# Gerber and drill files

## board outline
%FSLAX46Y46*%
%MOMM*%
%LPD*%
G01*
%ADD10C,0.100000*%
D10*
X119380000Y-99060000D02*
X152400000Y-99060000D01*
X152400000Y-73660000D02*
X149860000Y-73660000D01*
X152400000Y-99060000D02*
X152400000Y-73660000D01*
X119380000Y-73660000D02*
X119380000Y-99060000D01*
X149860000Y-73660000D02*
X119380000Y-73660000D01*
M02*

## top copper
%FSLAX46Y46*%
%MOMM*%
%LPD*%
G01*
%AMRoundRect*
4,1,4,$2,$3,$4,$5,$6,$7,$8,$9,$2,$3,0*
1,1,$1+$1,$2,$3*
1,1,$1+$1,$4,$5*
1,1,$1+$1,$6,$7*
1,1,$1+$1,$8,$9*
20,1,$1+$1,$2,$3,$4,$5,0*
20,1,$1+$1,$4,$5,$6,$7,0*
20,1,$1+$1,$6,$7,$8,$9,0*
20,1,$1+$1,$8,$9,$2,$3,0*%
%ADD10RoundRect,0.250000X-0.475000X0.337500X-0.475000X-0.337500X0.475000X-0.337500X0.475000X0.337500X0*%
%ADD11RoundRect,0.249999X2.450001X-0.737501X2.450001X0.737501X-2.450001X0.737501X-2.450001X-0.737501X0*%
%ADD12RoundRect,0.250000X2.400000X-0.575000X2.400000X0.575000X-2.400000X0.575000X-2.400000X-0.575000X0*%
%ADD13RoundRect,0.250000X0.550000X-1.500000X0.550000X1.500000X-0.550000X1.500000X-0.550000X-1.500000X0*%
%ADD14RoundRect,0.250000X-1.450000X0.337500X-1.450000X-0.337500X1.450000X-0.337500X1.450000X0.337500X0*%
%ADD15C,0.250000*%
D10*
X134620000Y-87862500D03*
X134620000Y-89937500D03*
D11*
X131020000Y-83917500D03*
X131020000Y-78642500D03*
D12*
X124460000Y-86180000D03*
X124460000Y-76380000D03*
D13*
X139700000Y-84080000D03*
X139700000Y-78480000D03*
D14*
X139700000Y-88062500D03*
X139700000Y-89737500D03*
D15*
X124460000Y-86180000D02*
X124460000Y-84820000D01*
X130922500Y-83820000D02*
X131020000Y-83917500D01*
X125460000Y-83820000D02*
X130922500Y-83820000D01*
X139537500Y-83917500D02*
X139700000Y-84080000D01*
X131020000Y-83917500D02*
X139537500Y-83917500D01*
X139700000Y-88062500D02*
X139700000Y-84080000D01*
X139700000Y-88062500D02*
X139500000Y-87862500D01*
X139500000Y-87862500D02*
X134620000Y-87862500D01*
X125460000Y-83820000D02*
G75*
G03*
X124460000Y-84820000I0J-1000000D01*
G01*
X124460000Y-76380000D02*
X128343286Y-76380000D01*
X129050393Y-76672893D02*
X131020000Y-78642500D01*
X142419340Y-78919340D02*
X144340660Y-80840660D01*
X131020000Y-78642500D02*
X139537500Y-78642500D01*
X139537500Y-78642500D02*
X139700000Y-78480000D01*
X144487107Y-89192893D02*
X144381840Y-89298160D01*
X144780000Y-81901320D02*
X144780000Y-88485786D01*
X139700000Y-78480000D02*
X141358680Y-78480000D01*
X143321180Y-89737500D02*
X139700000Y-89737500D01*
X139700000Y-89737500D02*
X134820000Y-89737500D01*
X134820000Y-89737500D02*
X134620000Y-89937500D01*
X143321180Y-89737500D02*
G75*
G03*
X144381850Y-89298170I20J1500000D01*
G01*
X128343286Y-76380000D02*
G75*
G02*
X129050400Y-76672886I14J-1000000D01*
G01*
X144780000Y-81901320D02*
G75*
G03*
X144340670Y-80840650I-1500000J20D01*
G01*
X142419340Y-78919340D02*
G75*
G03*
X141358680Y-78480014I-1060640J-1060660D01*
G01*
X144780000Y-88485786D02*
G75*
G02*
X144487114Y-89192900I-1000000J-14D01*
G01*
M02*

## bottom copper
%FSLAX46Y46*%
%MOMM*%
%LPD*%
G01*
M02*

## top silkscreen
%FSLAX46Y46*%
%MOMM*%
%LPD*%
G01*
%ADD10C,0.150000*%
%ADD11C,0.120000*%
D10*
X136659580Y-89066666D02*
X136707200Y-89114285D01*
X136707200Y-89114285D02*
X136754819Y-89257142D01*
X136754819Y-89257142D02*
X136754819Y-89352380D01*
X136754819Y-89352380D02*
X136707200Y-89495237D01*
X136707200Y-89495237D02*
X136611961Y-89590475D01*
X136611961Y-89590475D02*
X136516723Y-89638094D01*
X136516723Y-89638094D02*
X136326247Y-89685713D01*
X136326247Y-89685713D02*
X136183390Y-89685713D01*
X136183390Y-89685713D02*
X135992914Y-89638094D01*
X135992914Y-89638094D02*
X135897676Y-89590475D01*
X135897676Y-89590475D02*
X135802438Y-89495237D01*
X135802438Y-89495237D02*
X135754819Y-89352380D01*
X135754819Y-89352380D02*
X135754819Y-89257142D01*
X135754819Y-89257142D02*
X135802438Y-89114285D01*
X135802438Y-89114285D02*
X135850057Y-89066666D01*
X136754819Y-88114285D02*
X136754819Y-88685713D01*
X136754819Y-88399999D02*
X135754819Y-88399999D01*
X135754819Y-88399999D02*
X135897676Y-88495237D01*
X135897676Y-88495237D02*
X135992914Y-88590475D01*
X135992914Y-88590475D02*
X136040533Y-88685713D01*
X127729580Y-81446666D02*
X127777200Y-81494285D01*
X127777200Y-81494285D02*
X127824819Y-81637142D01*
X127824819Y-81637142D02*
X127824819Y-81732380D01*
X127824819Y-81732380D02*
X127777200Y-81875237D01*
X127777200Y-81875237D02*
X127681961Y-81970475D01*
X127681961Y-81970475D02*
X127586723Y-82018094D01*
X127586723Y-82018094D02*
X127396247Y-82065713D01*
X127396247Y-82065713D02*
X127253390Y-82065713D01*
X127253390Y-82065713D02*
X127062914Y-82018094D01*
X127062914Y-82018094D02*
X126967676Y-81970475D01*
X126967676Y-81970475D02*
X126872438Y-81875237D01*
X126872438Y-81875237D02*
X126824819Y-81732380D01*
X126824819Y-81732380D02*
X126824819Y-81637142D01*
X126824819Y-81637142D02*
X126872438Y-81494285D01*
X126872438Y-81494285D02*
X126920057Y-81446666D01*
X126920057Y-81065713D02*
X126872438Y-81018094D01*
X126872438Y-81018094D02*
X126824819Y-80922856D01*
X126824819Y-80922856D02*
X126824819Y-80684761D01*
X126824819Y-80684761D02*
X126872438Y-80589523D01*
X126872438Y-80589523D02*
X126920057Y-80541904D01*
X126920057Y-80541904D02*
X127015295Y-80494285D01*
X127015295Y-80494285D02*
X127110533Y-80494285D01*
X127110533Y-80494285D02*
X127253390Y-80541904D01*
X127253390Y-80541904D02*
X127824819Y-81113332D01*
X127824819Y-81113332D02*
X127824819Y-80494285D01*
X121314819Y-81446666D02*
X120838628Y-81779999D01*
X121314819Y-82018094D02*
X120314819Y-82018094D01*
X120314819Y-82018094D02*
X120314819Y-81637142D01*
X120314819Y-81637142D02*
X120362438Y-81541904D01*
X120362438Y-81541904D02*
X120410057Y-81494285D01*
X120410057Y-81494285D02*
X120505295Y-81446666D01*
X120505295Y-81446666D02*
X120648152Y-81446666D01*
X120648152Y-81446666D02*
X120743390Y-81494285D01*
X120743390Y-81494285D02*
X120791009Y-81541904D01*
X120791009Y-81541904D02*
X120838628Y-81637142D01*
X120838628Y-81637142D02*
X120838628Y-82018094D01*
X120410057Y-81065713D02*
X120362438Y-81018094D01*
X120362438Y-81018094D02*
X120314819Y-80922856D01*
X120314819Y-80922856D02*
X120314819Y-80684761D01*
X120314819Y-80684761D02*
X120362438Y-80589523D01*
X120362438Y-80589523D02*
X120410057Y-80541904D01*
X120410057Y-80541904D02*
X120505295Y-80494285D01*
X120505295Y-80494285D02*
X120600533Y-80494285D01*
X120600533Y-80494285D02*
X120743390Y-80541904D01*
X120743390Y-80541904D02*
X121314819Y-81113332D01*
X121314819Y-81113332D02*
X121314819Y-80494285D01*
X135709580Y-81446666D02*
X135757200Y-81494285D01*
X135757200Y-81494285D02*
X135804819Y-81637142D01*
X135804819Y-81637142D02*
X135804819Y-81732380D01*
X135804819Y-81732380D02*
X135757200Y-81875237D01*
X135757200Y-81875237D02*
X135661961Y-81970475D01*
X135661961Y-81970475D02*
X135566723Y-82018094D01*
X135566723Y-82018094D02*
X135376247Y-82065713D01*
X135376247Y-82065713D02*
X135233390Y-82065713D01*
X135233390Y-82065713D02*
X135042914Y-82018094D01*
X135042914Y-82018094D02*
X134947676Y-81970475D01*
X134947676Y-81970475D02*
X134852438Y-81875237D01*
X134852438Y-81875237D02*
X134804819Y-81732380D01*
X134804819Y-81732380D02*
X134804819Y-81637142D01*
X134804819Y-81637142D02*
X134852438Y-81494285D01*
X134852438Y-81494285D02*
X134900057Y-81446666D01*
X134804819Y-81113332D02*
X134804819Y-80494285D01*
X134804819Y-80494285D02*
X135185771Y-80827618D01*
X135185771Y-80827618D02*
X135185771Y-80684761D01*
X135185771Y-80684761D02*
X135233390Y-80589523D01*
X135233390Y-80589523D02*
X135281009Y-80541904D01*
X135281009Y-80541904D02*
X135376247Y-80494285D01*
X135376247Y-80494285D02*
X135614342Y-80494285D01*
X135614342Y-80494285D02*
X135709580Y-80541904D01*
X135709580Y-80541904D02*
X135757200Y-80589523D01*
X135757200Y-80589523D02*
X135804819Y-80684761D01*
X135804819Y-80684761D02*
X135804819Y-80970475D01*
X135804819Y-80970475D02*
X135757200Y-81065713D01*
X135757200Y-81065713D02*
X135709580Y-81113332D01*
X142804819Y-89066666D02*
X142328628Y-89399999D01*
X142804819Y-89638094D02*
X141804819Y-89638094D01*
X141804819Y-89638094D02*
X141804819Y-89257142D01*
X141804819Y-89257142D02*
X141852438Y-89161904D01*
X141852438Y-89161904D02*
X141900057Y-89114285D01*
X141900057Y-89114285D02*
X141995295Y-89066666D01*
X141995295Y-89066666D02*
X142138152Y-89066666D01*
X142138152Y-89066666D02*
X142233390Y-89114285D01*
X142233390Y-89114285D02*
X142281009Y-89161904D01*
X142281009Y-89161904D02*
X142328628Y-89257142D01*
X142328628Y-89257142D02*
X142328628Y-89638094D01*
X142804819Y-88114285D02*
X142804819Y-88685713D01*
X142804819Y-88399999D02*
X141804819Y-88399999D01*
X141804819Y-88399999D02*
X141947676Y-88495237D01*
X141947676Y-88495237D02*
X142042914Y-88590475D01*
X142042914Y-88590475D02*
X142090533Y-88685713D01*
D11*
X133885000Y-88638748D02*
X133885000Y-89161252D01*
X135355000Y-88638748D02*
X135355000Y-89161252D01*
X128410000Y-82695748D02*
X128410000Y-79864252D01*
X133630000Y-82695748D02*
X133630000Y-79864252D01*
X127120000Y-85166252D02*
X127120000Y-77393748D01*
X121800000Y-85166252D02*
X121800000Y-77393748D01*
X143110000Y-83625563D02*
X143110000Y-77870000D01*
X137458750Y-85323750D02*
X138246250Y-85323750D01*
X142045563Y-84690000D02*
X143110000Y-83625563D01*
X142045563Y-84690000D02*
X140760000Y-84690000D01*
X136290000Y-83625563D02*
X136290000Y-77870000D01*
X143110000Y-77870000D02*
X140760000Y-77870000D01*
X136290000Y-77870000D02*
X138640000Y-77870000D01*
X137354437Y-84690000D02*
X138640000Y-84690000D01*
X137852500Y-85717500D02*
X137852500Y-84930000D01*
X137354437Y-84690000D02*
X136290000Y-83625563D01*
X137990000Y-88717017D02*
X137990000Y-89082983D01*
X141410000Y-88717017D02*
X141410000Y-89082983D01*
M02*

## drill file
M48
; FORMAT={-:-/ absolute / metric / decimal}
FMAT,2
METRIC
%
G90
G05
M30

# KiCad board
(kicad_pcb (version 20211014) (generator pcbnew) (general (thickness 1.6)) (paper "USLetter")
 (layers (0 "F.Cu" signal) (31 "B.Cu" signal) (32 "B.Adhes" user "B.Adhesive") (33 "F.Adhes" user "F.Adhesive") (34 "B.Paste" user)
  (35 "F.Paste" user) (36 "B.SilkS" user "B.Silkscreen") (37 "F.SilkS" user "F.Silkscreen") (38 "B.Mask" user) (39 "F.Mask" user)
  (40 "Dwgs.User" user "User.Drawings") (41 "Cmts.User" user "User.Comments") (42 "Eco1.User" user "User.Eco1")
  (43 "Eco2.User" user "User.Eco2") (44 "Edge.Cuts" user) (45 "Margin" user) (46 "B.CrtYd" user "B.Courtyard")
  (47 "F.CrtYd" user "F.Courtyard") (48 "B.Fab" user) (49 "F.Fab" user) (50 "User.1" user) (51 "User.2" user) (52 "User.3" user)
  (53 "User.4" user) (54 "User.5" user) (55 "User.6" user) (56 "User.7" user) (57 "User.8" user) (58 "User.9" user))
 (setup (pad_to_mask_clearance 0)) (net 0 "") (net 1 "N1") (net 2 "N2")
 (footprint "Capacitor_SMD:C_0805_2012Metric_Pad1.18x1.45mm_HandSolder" (layer "F.Cu") (at 134.62 88.9 -90)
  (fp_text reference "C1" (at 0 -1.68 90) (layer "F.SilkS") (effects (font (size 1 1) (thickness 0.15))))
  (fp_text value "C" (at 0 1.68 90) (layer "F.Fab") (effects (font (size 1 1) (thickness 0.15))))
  (fp_line (start -0.261252 0.735) (end 0.261252 0.735) (layer "F.SilkS") (width 0.12))
  (fp_line (start -0.261252 -0.735) (end 0.261252 -0.735) (layer "F.SilkS") (width 0.12))
  (pad "1" smd roundrect (at -1.0375 0 270) (size 1.175 1.45) (layers "F.Cu" "F.Paste" "F.Mask") (roundrect_rratio 0.212766) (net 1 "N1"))
  (pad "2" smd roundrect (at 1.0375 0 270) (size 1.175 1.45) (layers "F.Cu" "F.Paste" "F.Mask") (roundrect_rratio 0.212766) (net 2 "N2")))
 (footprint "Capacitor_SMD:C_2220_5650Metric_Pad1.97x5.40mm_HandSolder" (layer "F.Cu") (at 131.02 81.28 90)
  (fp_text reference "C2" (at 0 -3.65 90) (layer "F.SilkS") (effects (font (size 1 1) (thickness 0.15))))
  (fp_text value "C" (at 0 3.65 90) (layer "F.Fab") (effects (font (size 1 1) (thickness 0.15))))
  (fp_line (start -1.415748 -2.61) (end 1.415748 -2.61) (layer "F.SilkS") (width 0.12))
  (fp_line (start -1.415748 2.61) (end 1.415748 2.61) (layer "F.SilkS") (width 0.12))
  (pad "1" smd roundrect (at -2.6375 0 90) (size 1.975 5.4) (layers "F.Cu" "F.Paste" "F.Mask") (roundrect_rratio 0.126582) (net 1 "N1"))
  (pad "2" smd roundrect (at 2.6375 0 90) (size 1.975 5.4) (layers "F.Cu" "F.Paste" "F.Mask") (roundrect_rratio 0.126582) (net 2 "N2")))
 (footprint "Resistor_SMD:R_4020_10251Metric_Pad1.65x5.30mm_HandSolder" (layer "F.Cu") (at 124.46 81.28 90)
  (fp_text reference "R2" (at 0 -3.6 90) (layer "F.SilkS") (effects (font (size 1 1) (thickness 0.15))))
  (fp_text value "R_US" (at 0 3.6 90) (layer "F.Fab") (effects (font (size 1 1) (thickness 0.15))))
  (fp_line (start -3.886252 2.66) (end 3.886252 2.66) (layer "F.SilkS") (width 0.12))
  (fp_line (start -3.886252 -2.66) (end 3.886252 -2.66) (layer "F.SilkS") (width 0.12))
  (pad "1" smd roundrect (at -4.9 0 90) (size 1.65 5.3) (layers "F.Cu" "F.Paste" "F.Mask") (roundrect_rratio 0.151515) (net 1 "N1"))
  (pad "2" smd roundrect (at 4.9 0 90) (size 1.65 5.3) (layers "F.Cu" "F.Paste" "F.Mask") (roundrect_rratio 0.151515) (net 2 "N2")))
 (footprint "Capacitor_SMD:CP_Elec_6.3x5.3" (layer "F.Cu") (at 139.7 81.28 90)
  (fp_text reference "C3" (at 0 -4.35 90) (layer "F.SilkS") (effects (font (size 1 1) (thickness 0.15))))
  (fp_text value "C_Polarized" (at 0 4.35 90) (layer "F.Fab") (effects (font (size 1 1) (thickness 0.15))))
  (fp_line (start -2.345563 3.41) (end 3.41 3.41) (layer "F.SilkS") (width 0.12))
  (fp_line (start -4.04375 -2.24125) (end -4.04375 -1.45375) (layer "F.SilkS") (width 0.12))
  (fp_line (start -3.41 2.345563) (end -2.345563 3.41) (layer "F.SilkS") (width 0.12))
  (fp_line (start -3.41 2.345563) (end -3.41 1.06) (layer "F.SilkS") (width 0.12))
  (fp_line (start -2.345563 -3.41) (end 3.41 -3.41) (layer "F.SilkS") (width 0.12))
  (fp_line (start 3.41 3.41) (end 3.41 1.06) (layer "F.SilkS") (width 0.12))
  (fp_line (start 3.41 -3.41) (end 3.41 -1.06) (layer "F.SilkS") (width 0.12))
  (fp_line (start -3.41 -2.345563) (end -3.41 -1.06) (layer "F.SilkS") (width 0.12))
  (fp_line (start -4.4375 -1.8475) (end -3.65 -1.8475) (layer "F.SilkS") (width 0.12))
  (fp_line (start -3.41 -2.345563) (end -2.345563 -3.41) (layer "F.SilkS") (width 0.12))
  (pad "1" smd roundrect (at -2.8 0 90) (size 3.5 1.6) (layers "F.Cu" "F.Paste" "F.Mask") (roundrect_rratio 0.15625) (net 1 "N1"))
  (pad "2" smd roundrect (at 2.8 0 90) (size 3.5 1.6) (layers "F.Cu" "F.Paste" "F.Mask") (roundrect_rratio 0.15625) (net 2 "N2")))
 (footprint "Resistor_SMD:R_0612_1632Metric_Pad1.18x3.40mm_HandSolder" (layer "F.Cu") (at 139.7 88.9 -90)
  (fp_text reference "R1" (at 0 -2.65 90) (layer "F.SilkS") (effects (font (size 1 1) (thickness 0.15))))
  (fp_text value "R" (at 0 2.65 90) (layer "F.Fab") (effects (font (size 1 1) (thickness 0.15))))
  (fp_line (start -0.182983 1.71) (end 0.182983 1.71) (layer "F.SilkS") (width 0.12))
  (fp_line (start -0.182983 -1.71) (end 0.182983 -1.71) (layer "F.SilkS") (width 0.12))
  (pad "1" smd roundrect (at -0.8375 0 270) (size 1.175 3.4) (layers "F.Cu" "F.Paste" "F.Mask") (roundrect_rratio 0.212766) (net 1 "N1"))
  (pad "2" smd roundrect (at 0.8375 0 270) (size 1.175 3.4) (layers "F.Cu" "F.Paste" "F.Mask") (roundrect_rratio 0.212766) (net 2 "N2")))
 (gr_line (start 119.38 99.06) (end 152.4 99.06) (layer "Edge.Cuts") (width 0.1))
 (gr_line (start 152.4 73.66) (end 149.86 73.66) (layer "Edge.Cuts") (width 0.1))
 (gr_line (start 152.4 99.06) (end 152.4 73.66) (layer "Edge.Cuts") (width 0.1))
 (gr_line (start 119.38 73.66) (end 119.38 99.06) (layer "Edge.Cuts") (width 0.1))
 (gr_line (start 149.86 73.66) (end 119.38 73.66) (layer "Edge.Cuts") (width 0.1))
 (segment (start 124.46 86.18) (end 124.46 84.82) (width 0.25) (layer "F.Cu") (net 1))
 (segment (start 130.9225 83.82) (end 131.02 83.9175) (width 0.25) (layer "F.Cu") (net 1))
 (segment (start 125.46 83.82) (end 130.9225 83.82) (width 0.25) (layer "F.Cu") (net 1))
 (segment (start 139.5375 83.9175) (end 139.7 84.08) (width 0.25) (layer "F.Cu") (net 1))
 (segment (start 131.02 83.9175) (end 139.5375 83.9175) (width 0.25) (layer "F.Cu") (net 1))
 (segment (start 139.7 88.0625) (end 139.7 84.08) (width 0.25) (layer "F.Cu") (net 1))
 (segment (start 139.7 88.0625) (end 139.5 87.8625) (width 0.25) (layer "F.Cu") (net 1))
 (segment (start 139.5 87.8625) (end 134.62 87.8625) (width 0.25) (layer "F.Cu") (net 1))
 (arc (start 125.46 83.82) (mid 124.752893 84.112893) (end 124.46 84.82) (width 0.25) (layer "F.Cu") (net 1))
 (segment (start 124.46 76.38) (end 128.343286 76.38) (width 0.25) (layer "F.Cu") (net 2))
 (segment (start 129.050393 76.672893) (end 131.02 78.6425) (width 0.25) (layer "F.Cu") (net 2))
 (segment (start 142.41934 78.91934) (end 144.34066 80.84066) (width 0.25) (layer "F.Cu") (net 2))
 (segment (start 131.02 78.6425) (end 139.5375 78.6425) (width 0.25) (layer "F.Cu") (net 2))
 (segment (start 139.5375 78.6425) (end 139.7 78.48) (width 0.25) (layer "F.Cu") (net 2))
 (segment (start 144.487107 89.192893) (end 144.38184 89.29816) (width 0.25) (layer "F.Cu") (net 2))
 (segment (start 144.78 81.90132) (end 144.78 88.485786) (width 0.25) (layer "F.Cu") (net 2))
 (segment (start 139.7 78.48) (end 141.35868 78.48) (width 0.25) (layer "F.Cu") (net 2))
 (segment (start 143.32118 89.7375) (end 139.7 89.7375) (width 0.25) (layer "F.Cu") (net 2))
 (segment (start 139.7 89.7375) (end 134.82 89.7375) (width 0.25) (layer "F.Cu") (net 2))
 (segment (start 134.82 89.7375) (end 134.62 89.9375) (width 0.25) (layer "F.Cu") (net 2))
 (arc (start 143.32118 89.7375) (mid 143.895205 89.623319) (end 144.38184 89.29816) (width 0.25) (layer "F.Cu") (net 2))
 (arc (start 128.343286 76.38) (mid 128.725969 76.45612) (end 129.050393 76.672893) (width 0.25) (layer "F.Cu") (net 2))
 (arc (start 144.78 81.90132) (mid 144.665819 81.327295) (end 144.34066 80.84066) (width 0.25) (layer "F.Cu") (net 2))
 (arc (start 142.41934 78.91934) (mid 141.932705 78.594181) (end 141.35868 78.48) (width 0.25) (layer "F.Cu") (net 2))
 (arc (start 144.78 88.485786) (mid 144.70388 88.868469) (end 144.487107 89.192893) (width 0.25) (layer "F.Cu") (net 2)))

